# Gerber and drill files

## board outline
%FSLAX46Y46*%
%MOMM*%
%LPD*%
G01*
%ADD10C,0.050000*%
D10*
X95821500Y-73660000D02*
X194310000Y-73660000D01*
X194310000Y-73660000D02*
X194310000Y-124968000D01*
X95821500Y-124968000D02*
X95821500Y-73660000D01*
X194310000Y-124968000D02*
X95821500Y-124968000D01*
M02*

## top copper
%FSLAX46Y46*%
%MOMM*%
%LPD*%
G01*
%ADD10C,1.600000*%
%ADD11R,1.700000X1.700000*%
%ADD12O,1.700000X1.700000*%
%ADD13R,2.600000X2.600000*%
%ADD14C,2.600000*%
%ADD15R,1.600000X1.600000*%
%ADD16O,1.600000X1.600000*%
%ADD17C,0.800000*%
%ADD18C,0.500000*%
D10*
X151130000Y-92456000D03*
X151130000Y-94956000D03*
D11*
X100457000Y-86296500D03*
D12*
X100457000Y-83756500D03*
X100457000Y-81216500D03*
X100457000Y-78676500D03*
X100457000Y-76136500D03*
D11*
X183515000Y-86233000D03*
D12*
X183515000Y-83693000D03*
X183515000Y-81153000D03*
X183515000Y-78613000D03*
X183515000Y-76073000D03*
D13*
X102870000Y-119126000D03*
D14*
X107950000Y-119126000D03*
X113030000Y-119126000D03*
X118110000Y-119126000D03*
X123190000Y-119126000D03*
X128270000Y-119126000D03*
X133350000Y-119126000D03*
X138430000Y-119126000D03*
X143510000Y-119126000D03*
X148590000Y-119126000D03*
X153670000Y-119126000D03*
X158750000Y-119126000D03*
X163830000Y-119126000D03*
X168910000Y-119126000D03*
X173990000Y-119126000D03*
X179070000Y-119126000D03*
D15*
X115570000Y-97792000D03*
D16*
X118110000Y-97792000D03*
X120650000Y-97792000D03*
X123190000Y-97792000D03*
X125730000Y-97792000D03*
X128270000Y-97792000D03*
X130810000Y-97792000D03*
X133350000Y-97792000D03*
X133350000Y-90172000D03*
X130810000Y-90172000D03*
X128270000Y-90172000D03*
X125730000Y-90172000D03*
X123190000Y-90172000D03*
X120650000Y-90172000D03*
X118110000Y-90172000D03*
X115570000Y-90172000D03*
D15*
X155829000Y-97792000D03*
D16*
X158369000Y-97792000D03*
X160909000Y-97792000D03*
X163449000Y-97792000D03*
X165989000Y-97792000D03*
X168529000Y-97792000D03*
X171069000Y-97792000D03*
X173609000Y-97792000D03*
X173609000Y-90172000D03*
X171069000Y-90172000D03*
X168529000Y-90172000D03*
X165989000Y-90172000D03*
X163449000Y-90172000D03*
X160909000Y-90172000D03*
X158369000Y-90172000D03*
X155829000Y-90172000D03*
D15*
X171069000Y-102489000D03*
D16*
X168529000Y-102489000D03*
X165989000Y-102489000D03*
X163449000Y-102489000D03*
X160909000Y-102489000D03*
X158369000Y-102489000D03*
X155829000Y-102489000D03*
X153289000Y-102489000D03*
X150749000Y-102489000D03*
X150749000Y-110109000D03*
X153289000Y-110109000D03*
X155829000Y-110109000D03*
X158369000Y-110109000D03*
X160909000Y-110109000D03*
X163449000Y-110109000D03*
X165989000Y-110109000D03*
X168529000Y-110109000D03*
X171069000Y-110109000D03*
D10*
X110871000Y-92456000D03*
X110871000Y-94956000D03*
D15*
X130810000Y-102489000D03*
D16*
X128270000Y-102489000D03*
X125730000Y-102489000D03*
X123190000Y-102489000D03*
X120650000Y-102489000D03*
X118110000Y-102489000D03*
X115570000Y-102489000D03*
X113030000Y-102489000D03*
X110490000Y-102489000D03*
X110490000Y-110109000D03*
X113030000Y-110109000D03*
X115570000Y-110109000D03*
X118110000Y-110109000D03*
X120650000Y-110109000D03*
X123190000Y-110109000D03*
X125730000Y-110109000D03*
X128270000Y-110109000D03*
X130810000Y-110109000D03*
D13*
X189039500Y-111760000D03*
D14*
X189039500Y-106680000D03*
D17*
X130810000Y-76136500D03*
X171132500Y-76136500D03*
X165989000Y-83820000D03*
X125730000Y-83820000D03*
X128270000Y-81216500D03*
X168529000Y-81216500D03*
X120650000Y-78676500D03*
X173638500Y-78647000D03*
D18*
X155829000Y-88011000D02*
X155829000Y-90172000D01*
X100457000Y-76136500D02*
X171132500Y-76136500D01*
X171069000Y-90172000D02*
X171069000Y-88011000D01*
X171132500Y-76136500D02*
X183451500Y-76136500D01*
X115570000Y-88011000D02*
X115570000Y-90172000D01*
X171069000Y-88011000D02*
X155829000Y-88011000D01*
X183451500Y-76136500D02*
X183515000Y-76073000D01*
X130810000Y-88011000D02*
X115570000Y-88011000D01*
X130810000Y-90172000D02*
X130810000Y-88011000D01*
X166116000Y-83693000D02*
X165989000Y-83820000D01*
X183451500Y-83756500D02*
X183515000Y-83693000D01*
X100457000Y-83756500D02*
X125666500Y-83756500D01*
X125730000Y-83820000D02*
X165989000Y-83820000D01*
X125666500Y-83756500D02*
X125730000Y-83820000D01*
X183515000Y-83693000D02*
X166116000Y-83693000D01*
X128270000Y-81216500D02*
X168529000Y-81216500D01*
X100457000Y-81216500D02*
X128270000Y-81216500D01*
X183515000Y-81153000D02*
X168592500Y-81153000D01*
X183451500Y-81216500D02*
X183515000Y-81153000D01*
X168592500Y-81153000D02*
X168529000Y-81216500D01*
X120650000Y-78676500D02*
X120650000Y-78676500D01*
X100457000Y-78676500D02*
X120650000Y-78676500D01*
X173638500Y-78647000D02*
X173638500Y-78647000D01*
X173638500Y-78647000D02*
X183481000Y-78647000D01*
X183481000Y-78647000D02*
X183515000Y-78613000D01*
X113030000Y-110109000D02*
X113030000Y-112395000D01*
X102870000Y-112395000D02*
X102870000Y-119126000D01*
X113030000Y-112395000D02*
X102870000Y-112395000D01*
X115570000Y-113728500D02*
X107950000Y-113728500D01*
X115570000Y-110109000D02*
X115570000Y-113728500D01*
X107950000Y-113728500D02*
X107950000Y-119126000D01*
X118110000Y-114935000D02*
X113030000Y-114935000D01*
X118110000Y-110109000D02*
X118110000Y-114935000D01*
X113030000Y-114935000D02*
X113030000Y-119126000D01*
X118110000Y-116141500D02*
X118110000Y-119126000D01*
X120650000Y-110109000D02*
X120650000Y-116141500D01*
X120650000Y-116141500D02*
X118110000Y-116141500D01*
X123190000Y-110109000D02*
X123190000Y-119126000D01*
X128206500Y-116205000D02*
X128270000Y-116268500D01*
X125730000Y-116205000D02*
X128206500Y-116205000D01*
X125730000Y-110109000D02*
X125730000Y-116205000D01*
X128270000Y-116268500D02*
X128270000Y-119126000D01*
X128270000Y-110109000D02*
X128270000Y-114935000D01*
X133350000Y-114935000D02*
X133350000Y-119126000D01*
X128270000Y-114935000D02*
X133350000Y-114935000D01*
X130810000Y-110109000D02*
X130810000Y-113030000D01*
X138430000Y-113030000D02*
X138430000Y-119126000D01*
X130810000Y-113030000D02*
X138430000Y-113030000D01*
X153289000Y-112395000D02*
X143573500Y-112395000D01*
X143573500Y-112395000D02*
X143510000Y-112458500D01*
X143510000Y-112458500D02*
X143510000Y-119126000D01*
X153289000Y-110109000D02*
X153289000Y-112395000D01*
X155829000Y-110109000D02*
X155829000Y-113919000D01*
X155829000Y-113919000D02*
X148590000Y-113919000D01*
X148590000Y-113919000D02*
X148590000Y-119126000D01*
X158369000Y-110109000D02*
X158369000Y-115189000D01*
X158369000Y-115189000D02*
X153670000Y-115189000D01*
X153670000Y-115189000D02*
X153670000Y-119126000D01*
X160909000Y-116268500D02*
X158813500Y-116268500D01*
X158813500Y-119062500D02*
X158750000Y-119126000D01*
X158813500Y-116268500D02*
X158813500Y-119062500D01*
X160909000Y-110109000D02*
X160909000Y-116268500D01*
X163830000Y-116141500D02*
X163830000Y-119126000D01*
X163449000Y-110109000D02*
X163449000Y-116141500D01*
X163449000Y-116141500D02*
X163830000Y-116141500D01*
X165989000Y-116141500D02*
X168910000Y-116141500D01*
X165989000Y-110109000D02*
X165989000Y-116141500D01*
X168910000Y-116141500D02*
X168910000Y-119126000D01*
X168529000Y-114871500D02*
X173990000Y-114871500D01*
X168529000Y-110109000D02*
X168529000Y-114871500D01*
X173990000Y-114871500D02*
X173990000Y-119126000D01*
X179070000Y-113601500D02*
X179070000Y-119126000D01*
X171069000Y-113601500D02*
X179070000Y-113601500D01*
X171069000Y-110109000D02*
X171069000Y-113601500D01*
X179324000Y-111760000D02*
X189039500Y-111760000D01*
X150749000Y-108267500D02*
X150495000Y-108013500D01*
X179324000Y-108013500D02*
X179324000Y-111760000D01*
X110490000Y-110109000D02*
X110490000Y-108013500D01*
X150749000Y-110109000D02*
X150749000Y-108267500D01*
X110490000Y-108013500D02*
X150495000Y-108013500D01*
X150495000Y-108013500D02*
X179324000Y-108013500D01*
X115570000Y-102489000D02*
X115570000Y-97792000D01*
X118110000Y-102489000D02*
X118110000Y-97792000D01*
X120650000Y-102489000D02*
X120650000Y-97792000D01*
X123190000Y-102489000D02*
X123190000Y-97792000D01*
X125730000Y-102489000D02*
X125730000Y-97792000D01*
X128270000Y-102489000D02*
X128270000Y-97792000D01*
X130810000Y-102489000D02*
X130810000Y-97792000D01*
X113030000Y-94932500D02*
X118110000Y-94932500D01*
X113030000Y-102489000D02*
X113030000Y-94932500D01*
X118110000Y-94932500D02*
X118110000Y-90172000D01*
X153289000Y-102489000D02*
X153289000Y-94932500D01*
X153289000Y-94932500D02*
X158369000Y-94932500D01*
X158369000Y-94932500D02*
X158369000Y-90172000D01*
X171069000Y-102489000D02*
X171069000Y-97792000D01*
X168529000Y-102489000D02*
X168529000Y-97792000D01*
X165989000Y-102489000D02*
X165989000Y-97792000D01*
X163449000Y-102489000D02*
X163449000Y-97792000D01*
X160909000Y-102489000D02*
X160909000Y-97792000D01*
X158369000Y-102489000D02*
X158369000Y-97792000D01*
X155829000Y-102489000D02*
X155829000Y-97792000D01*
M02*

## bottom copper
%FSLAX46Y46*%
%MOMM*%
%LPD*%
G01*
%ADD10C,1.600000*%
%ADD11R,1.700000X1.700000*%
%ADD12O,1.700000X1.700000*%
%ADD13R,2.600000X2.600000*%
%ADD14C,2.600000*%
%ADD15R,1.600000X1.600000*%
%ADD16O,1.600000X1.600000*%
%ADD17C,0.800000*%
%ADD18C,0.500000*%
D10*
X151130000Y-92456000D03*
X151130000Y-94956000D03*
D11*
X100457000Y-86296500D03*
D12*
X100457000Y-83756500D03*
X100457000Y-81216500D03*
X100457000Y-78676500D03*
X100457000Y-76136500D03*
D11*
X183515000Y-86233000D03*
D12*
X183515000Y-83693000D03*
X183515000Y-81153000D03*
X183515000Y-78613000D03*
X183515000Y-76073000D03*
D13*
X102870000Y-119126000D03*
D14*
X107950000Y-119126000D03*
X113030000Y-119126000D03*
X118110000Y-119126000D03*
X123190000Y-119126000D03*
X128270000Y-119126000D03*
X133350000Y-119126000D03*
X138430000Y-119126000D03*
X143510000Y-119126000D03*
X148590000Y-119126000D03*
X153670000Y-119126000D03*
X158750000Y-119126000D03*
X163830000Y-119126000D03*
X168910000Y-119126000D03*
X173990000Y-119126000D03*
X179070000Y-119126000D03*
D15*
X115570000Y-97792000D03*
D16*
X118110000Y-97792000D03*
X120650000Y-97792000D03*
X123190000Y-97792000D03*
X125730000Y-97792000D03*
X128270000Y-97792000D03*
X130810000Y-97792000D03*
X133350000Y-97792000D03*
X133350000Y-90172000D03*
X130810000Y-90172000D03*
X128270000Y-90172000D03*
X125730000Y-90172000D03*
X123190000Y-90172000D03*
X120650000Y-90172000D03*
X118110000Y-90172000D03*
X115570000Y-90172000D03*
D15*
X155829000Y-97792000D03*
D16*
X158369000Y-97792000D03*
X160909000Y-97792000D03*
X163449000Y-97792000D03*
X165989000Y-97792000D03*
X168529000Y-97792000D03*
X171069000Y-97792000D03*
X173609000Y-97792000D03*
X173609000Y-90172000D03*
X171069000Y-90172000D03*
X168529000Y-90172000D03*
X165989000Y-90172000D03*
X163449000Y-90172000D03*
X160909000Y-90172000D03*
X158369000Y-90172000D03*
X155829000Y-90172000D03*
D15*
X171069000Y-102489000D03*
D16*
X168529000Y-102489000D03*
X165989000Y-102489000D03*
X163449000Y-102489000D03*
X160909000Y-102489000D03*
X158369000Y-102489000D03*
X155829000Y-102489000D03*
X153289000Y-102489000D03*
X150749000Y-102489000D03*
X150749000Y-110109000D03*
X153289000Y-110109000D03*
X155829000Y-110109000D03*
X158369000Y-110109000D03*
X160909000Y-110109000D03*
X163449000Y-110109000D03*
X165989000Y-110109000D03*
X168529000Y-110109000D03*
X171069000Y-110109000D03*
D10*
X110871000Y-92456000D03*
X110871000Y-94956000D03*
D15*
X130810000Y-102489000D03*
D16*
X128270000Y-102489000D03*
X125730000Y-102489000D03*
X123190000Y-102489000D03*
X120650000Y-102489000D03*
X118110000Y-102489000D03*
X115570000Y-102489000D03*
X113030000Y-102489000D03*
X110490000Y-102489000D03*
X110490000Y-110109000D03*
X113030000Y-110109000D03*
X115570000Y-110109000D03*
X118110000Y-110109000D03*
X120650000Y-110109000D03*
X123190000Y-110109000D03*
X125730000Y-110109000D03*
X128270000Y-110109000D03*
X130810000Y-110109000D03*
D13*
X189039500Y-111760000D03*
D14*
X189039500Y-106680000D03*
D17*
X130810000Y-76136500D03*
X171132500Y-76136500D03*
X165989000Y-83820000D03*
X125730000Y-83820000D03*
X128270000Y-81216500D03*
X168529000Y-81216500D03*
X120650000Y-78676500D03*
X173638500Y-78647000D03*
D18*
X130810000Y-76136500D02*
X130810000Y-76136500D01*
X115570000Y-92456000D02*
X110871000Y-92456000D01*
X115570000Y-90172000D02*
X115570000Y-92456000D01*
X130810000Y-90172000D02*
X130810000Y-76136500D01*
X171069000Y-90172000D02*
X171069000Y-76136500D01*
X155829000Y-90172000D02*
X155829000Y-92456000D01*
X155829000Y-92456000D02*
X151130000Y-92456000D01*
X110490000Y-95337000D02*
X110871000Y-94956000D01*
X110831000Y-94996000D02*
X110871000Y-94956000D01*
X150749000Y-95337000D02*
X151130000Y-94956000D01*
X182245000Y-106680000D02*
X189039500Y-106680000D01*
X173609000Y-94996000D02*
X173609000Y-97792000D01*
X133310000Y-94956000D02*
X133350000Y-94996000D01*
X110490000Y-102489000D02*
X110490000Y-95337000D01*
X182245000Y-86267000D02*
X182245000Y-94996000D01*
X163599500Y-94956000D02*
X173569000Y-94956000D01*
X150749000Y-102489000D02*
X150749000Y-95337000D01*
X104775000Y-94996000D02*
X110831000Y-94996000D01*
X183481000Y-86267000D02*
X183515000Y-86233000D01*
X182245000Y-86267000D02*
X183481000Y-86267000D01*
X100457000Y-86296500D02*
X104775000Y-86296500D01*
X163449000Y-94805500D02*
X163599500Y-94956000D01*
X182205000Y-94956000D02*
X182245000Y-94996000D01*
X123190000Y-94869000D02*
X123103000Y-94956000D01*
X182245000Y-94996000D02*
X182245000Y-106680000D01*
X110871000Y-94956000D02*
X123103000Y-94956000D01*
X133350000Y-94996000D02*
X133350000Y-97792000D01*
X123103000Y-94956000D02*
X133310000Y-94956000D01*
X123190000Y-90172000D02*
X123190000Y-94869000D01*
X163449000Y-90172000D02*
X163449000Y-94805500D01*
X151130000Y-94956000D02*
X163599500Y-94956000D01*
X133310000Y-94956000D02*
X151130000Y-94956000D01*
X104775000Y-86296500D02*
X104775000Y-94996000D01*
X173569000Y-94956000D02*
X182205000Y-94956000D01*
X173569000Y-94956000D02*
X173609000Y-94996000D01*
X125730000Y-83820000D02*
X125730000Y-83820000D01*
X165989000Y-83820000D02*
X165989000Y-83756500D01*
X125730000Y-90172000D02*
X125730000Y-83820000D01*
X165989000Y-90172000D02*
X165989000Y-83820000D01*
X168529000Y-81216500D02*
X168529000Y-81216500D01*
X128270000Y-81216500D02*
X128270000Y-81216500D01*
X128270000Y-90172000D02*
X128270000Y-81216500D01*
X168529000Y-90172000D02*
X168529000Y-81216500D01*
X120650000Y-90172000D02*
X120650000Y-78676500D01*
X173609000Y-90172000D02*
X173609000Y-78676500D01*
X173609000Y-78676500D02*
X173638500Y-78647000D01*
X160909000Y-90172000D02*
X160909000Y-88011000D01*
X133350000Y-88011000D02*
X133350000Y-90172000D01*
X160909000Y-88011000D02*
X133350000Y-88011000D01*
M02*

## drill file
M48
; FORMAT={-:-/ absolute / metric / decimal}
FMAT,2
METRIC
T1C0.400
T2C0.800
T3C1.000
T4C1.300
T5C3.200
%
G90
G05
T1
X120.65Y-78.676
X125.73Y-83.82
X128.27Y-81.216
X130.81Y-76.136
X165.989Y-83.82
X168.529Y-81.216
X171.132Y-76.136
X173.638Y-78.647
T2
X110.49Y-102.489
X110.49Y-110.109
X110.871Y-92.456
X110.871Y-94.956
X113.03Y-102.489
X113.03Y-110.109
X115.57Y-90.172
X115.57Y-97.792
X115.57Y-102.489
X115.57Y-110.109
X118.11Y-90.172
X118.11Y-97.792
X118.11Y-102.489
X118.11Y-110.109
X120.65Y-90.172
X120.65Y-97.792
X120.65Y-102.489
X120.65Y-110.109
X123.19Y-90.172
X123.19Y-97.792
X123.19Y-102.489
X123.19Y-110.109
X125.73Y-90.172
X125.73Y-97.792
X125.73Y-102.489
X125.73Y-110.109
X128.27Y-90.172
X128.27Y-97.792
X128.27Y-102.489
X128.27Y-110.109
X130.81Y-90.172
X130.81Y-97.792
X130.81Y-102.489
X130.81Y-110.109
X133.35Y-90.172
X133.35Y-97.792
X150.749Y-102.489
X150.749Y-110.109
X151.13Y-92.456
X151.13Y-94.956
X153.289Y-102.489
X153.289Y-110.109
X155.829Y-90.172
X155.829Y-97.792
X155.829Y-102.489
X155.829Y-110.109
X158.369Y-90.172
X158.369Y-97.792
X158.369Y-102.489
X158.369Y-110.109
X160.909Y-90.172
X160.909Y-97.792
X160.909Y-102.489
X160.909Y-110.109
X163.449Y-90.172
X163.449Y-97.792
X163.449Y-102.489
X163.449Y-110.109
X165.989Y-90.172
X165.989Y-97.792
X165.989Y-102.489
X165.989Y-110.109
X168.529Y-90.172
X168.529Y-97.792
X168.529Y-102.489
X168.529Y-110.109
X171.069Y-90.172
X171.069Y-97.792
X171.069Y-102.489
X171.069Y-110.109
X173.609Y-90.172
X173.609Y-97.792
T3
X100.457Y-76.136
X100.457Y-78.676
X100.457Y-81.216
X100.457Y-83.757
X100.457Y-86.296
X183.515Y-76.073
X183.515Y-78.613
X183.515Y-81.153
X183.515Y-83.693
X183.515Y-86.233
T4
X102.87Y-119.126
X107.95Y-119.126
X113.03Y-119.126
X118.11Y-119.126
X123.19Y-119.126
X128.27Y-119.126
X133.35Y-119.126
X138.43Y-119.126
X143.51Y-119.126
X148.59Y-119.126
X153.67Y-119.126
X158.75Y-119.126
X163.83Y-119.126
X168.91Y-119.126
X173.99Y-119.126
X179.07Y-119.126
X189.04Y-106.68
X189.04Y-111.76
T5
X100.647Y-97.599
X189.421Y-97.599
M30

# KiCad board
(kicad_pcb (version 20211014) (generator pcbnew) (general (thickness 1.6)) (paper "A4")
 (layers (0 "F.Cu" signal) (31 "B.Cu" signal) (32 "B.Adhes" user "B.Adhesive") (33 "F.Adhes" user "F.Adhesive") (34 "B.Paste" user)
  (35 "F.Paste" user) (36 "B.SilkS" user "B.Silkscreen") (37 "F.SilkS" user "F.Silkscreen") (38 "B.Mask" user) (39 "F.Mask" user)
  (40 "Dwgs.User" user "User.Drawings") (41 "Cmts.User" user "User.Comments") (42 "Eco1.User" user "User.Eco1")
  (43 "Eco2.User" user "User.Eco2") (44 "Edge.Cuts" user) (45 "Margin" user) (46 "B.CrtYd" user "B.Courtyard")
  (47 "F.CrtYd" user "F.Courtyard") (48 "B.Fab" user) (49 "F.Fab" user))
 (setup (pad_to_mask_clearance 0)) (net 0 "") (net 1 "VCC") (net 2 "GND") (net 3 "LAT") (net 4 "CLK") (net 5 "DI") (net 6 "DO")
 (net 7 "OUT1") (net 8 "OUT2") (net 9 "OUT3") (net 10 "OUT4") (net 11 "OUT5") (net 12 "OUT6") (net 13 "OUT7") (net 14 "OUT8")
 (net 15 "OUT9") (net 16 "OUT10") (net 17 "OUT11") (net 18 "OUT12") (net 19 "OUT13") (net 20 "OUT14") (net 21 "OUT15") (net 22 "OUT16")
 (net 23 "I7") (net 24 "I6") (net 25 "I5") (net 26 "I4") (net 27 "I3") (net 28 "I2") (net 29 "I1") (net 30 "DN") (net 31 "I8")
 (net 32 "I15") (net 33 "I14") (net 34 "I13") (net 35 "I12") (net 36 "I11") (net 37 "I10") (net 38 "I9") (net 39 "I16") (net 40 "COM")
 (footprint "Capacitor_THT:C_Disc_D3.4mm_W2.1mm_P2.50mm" (layer "F.Cu") (at 151.13 92.456 -90)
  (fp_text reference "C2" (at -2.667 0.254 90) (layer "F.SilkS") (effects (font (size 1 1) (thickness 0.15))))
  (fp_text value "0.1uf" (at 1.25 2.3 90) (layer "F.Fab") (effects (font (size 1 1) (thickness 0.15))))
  (pad "1" thru_hole circle locked (at 0 0 270) (size 1.6 1.6) (drill 0.8) (layers *.Cu *.Mask) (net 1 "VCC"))
  (pad "2" thru_hole circle locked (at 2.5 0 270) (size 1.6 1.6) (drill 0.8) (layers *.Cu *.Mask) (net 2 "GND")))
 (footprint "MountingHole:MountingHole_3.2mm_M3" (layer "F.Cu") (at 100.6475 97.5995)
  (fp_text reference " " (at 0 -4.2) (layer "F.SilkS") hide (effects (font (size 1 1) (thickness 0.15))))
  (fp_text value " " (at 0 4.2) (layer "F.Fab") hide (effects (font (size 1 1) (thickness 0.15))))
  (pad "" np_thru_hole circle locked (at 0 0) (size 3.2 3.2) (drill 3.2) (layers *.Cu *.Mask)))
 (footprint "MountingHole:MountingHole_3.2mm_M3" (layer "F.Cu") (at 189.4205 97.5995)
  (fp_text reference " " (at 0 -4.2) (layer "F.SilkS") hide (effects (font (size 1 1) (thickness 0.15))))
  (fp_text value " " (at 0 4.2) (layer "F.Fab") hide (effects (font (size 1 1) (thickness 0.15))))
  (pad "" np_thru_hole circle locked (at 0 0) (size 3.2 3.2) (drill 3.2) (layers *.Cu *.Mask)))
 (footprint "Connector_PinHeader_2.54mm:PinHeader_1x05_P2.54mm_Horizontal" (layer "F.Cu") (at 100.457 86.2965 180)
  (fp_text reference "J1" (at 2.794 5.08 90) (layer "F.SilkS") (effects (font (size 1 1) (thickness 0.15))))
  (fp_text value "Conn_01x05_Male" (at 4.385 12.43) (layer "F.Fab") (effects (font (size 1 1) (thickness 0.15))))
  (pad "1" thru_hole rect locked (at 0 0 180) (size 1.7 1.7) (drill 1) (layers *.Cu *.Mask) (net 2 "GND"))
  (pad "2" thru_hole oval locked (at 0 2.54 180) (size 1.7 1.7) (drill 1) (layers *.Cu *.Mask) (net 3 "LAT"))
  (pad "3" thru_hole oval locked (at 0 5.08 180) (size 1.7 1.7) (drill 1) (layers *.Cu *.Mask) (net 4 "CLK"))
  (pad "4" thru_hole oval locked (at 0 7.62 180) (size 1.7 1.7) (drill 1) (layers *.Cu *.Mask) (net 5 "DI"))
  (pad "5" thru_hole oval locked (at 0 10.16 180) (size 1.7 1.7) (drill 1) (layers *.Cu *.Mask) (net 1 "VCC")))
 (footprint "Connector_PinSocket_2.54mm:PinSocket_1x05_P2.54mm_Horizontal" (layer "F.Cu") (at 183.515 86.233 180)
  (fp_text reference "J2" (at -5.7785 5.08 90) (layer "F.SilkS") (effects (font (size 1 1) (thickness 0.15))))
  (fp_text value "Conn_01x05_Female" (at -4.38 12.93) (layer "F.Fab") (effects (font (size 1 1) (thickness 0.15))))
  (pad "1" thru_hole rect locked (at 0 0 180) (size 1.7 1.7) (drill 1) (layers *.Cu *.Mask) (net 2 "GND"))
  (pad "2" thru_hole oval locked (at 0 2.54 180) (size 1.7 1.7) (drill 1) (layers *.Cu *.Mask) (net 3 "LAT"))
  (pad "3" thru_hole oval locked (at 0 5.08 180) (size 1.7 1.7) (drill 1) (layers *.Cu *.Mask) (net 4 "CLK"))
  (pad "4" thru_hole oval locked (at 0 7.62 180) (size 1.7 1.7) (drill 1) (layers *.Cu *.Mask) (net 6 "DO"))
  (pad "5" thru_hole oval locked (at 0 10.16 180) (size 1.7 1.7) (drill 1) (layers *.Cu *.Mask) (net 1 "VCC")))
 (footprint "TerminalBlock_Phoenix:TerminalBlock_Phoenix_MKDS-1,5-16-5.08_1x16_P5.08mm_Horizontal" (layer "F.Cu") (at 102.87 119.126)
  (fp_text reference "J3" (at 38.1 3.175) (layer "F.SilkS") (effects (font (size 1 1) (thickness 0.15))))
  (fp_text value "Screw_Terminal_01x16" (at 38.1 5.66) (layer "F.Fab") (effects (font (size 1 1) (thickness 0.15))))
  (pad "1" thru_hole rect locked (at 0 0) (size 2.6 2.6) (drill 1.3) (layers *.Cu *.Mask) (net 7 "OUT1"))
  (pad "2" thru_hole circle locked (at 5.08 0) (size 2.6 2.6) (drill 1.3) (layers *.Cu *.Mask) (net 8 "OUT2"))
  (pad "3" thru_hole circle locked (at 10.16 0) (size 2.6 2.6) (drill 1.3) (layers *.Cu *.Mask) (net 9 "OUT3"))
  (pad "4" thru_hole circle locked (at 15.24 0) (size 2.6 2.6) (drill 1.3) (layers *.Cu *.Mask) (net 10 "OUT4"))
  (pad "5" thru_hole circle locked (at 20.32 0) (size 2.6 2.6) (drill 1.3) (layers *.Cu *.Mask) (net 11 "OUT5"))
  (pad "6" thru_hole circle locked (at 25.4 0) (size 2.6 2.6) (drill 1.3) (layers *.Cu *.Mask) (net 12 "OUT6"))
  (pad "7" thru_hole circle locked (at 30.48 0) (size 2.6 2.6) (drill 1.3) (layers *.Cu *.Mask) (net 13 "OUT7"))
  (pad "8" thru_hole circle locked (at 35.56 0) (size 2.6 2.6) (drill 1.3) (layers *.Cu *.Mask) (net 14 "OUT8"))
  (pad "9" thru_hole circle locked (at 40.64 0) (size 2.6 2.6) (drill 1.3) (layers *.Cu *.Mask) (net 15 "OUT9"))
  (pad "10" thru_hole circle locked (at 45.72 0) (size 2.6 2.6) (drill 1.3) (layers *.Cu *.Mask) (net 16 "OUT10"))
  (pad "11" thru_hole circle locked (at 50.8 0) (size 2.6 2.6) (drill 1.3) (layers *.Cu *.Mask) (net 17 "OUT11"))
  (pad "12" thru_hole circle locked (at 55.88 0) (size 2.6 2.6) (drill 1.3) (layers *.Cu *.Mask) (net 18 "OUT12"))
  (pad "13" thru_hole circle locked (at 60.96 0) (size 2.6 2.6) (drill 1.3) (layers *.Cu *.Mask) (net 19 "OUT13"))
  (pad "14" thru_hole circle locked (at 66.04 0) (size 2.6 2.6) (drill 1.3) (layers *.Cu *.Mask) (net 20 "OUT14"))
  (pad "15" thru_hole circle locked (at 71.12 0) (size 2.6 2.6) (drill 1.3) (layers *.Cu *.Mask) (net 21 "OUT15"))
  (pad "16" thru_hole circle locked (at 76.2 0) (size 2.6 2.6) (drill 1.3) (layers *.Cu *.Mask) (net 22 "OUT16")))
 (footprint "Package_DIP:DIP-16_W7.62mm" (layer "F.Cu") (at 115.57 97.792 90)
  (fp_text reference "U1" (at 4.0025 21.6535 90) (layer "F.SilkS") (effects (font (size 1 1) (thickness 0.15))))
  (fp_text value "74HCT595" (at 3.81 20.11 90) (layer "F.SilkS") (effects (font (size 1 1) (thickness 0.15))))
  (pad "1" thru_hole rect locked (at 0 0 90) (size 1.6 1.6) (drill 0.8) (layers *.Cu *.Mask) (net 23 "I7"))
  (pad "2" thru_hole oval locked (at 0 2.54 90) (size 1.6 1.6) (drill 0.8) (layers *.Cu *.Mask) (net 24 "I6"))
  (pad "3" thru_hole oval locked (at 0 5.08 90) (size 1.6 1.6) (drill 0.8) (layers *.Cu *.Mask) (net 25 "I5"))
  (pad "4" thru_hole oval locked (at 0 7.62 90) (size 1.6 1.6) (drill 0.8) (layers *.Cu *.Mask) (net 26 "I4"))
  (pad "5" thru_hole oval locked (at 0 10.16 90) (size 1.6 1.6) (drill 0.8) (layers *.Cu *.Mask) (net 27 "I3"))
  (pad "6" thru_hole oval locked (at 0 12.7 90) (size 1.6 1.6) (drill 0.8) (layers *.Cu *.Mask) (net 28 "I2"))
  (pad "7" thru_hole oval locked (at 0 15.24 90) (size 1.6 1.6) (drill 0.8) (layers *.Cu *.Mask) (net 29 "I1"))
  (pad "8" thru_hole oval locked (at 0 17.78 90) (size 1.6 1.6) (drill 0.8) (layers *.Cu *.Mask) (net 2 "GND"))
  (pad "9" thru_hole oval locked (at 7.62 17.78 90) (size 1.6 1.6) (drill 0.8) (layers *.Cu *.Mask) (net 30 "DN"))
  (pad "10" thru_hole oval locked (at 7.62 15.24 90) (size 1.6 1.6) (drill 0.8) (layers *.Cu *.Mask) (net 1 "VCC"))
  (pad "11" thru_hole oval locked (at 7.62 12.7 90) (size 1.6 1.6) (drill 0.8) (layers *.Cu *.Mask) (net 4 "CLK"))
  (pad "12" thru_hole oval locked (at 7.62 10.16 90) (size 1.6 1.6) (drill 0.8) (layers *.Cu *.Mask) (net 3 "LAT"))
  (pad "13" thru_hole oval locked (at 7.62 7.62 90) (size 1.6 1.6) (drill 0.8) (layers *.Cu *.Mask) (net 2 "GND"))
  (pad "14" thru_hole oval locked (at 7.62 5.08 90) (size 1.6 1.6) (drill 0.8) (layers *.Cu *.Mask) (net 5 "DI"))
  (pad "15" thru_hole oval locked (at 7.62 2.54 90) (size 1.6 1.6) (drill 0.8) (layers *.Cu *.Mask) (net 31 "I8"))
  (pad "16" thru_hole oval locked (at 7.62 0 90) (size 1.6 1.6) (drill 0.8) (layers *.Cu *.Mask) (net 1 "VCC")))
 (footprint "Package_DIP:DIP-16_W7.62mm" (layer "F.Cu") (at 155.829 97.792 90)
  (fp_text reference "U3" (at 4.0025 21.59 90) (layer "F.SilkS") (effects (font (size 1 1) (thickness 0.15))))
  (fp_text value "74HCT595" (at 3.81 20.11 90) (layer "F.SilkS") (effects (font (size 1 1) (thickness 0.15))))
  (pad "1" thru_hole rect locked (at 0 0 90) (size 1.6 1.6) (drill 0.8) (layers *.Cu *.Mask) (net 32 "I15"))
  (pad "2" thru_hole oval locked (at 0 2.54 90) (size 1.6 1.6) (drill 0.8) (layers *.Cu *.Mask) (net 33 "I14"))
  (pad "3" thru_hole oval locked (at 0 5.08 90) (size 1.6 1.6) (drill 0.8) (layers *.Cu *.Mask) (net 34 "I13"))
  (pad "4" thru_hole oval locked (at 0 7.62 90) (size 1.6 1.6) (drill 0.8) (layers *.Cu *.Mask) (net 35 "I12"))
  (pad "5" thru_hole oval locked (at 0 10.16 90) (size 1.6 1.6) (drill 0.8) (layers *.Cu *.Mask) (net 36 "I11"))
  (pad "6" thru_hole oval locked (at 0 12.7 90) (size 1.6 1.6) (drill 0.8) (layers *.Cu *.Mask) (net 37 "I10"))
  (pad "7" thru_hole oval locked (at 0 15.24 90) (size 1.6 1.6) (drill 0.8) (layers *.Cu *.Mask) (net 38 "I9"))
  (pad "8" thru_hole oval locked (at 0 17.78 90) (size 1.6 1.6) (drill 0.8) (layers *.Cu *.Mask) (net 2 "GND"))
  (pad "9" thru_hole oval locked (at 7.62 17.78 90) (size 1.6 1.6) (drill 0.8) (layers *.Cu *.Mask) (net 6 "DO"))
  (pad "10" thru_hole oval locked (at 7.62 15.24 90) (size 1.6 1.6) (drill 0.8) (layers *.Cu *.Mask) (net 1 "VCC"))
  (pad "11" thru_hole oval locked (at 7.62 12.7 90) (size 1.6 1.6) (drill 0.8) (layers *.Cu *.Mask) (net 4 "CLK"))
  (pad "12" thru_hole oval locked (at 7.62 10.16 90) (size 1.6 1.6) (drill 0.8) (layers *.Cu *.Mask) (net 3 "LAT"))
  (pad "13" thru_hole oval locked (at 7.62 7.62 90) (size 1.6 1.6) (drill 0.8) (layers *.Cu *.Mask) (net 2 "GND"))
  (pad "14" thru_hole oval locked (at 7.62 5.08 90) (size 1.6 1.6) (drill 0.8) (layers *.Cu *.Mask) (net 30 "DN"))
  (pad "15" thru_hole oval locked (at 7.62 2.54 90) (size 1.6 1.6) (drill 0.8) (layers *.Cu *.Mask) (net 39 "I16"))
  (pad "16" thru_hole oval locked (at 7.62 0 90) (size 1.6 1.6) (drill 0.8) (layers *.Cu *.Mask) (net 1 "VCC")))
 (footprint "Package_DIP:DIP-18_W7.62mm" (layer "F.Cu") (at 171.069 102.489 -90)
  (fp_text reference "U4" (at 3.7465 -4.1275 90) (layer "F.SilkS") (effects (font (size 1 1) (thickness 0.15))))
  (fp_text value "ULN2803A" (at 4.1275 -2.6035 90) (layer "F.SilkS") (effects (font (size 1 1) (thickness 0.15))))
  (pad "1" thru_hole rect locked (at 0 0 270) (size 1.6 1.6) (drill 0.8) (layers *.Cu *.Mask) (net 38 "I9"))
  (pad "2" thru_hole oval locked (at 0 2.54 270) (size 1.6 1.6) (drill 0.8) (layers *.Cu *.Mask) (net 37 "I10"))
  (pad "3" thru_hole oval locked (at 0 5.08 270) (size 1.6 1.6) (drill 0.8) (layers *.Cu *.Mask) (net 36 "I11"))
  (pad "4" thru_hole oval locked (at 0 7.62 270) (size 1.6 1.6) (drill 0.8) (layers *.Cu *.Mask) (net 35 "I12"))
  (pad "5" thru_hole oval locked (at 0 10.16 270) (size 1.6 1.6) (drill 0.8) (layers *.Cu *.Mask) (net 34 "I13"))
  (pad "6" thru_hole oval locked (at 0 12.7 270) (size 1.6 1.6) (drill 0.8) (layers *.Cu *.Mask) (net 33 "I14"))
  (pad "7" thru_hole oval locked (at 0 15.24 270) (size 1.6 1.6) (drill 0.8) (layers *.Cu *.Mask) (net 32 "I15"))
  (pad "8" thru_hole oval locked (at 0 17.78 270) (size 1.6 1.6) (drill 0.8) (layers *.Cu *.Mask) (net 39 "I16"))
  (pad "9" thru_hole oval locked (at 0 20.32 270) (size 1.6 1.6) (drill 0.8) (layers *.Cu *.Mask) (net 2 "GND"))
  (pad "10" thru_hole oval locked (at 7.62 20.32 270) (size 1.6 1.6) (drill 0.8) (layers *.Cu *.Mask) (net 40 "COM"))
  (pad "11" thru_hole oval locked (at 7.62 17.78 270) (size 1.6 1.6) (drill 0.8) (layers *.Cu *.Mask) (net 15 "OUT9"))
  (pad "12" thru_hole oval locked (at 7.62 15.24 270) (size 1.6 1.6) (drill 0.8) (layers *.Cu *.Mask) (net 16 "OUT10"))
  (pad "13" thru_hole oval locked (at 7.62 12.7 270) (size 1.6 1.6) (drill 0.8) (layers *.Cu *.Mask) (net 17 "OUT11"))
  (pad "14" thru_hole oval locked (at 7.62 10.16 270) (size 1.6 1.6) (drill 0.8) (layers *.Cu *.Mask) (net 18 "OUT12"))
  (pad "15" thru_hole oval locked (at 7.62 7.62 270) (size 1.6 1.6) (drill 0.8) (layers *.Cu *.Mask) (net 19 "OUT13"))
  (pad "16" thru_hole oval locked (at 7.62 5.08 270) (size 1.6 1.6) (drill 0.8) (layers *.Cu *.Mask) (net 20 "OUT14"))
  (pad "17" thru_hole oval locked (at 7.62 2.54 270) (size 1.6 1.6) (drill 0.8) (layers *.Cu *.Mask) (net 21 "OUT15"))
  (pad "18" thru_hole oval locked (at 7.62 0 270) (size 1.6 1.6) (drill 0.8) (layers *.Cu *.Mask) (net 22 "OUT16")))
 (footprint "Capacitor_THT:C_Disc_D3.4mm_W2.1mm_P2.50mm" (layer "F.Cu") (at 110.871 92.456 -90)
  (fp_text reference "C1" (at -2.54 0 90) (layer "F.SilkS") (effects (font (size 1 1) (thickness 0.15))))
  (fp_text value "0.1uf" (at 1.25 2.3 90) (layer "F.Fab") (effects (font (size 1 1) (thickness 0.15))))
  (pad "1" thru_hole circle locked (at 0 0 270) (size 1.6 1.6) (drill 0.8) (layers *.Cu *.Mask) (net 1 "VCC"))
  (pad "2" thru_hole circle locked (at 2.5 0 270) (size 1.6 1.6) (drill 0.8) (layers *.Cu *.Mask) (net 2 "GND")))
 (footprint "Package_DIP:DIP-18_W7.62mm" (layer "F.Cu") (at 130.81 102.489 -90)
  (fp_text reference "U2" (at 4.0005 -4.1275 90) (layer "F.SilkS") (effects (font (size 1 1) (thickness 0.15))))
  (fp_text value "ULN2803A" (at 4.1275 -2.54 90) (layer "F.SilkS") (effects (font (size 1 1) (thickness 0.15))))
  (pad "1" thru_hole rect locked (at 0 0 270) (size 1.6 1.6) (drill 0.8) (layers *.Cu *.Mask) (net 29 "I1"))
  (pad "2" thru_hole oval locked (at 0 2.54 270) (size 1.6 1.6) (drill 0.8) (layers *.Cu *.Mask) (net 28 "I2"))
  (pad "3" thru_hole oval locked (at 0 5.08 270) (size 1.6 1.6) (drill 0.8) (layers *.Cu *.Mask) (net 27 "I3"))
  (pad "4" thru_hole oval locked (at 0 7.62 270) (size 1.6 1.6) (drill 0.8) (layers *.Cu *.Mask) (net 26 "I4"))
  (pad "5" thru_hole oval locked (at 0 10.16 270) (size 1.6 1.6) (drill 0.8) (layers *.Cu *.Mask) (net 25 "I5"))
  (pad "6" thru_hole oval locked (at 0 12.7 270) (size 1.6 1.6) (drill 0.8) (layers *.Cu *.Mask) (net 24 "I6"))
  (pad "7" thru_hole oval locked (at 0 15.24 270) (size 1.6 1.6) (drill 0.8) (layers *.Cu *.Mask) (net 23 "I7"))
  (pad "8" thru_hole oval locked (at 0 17.78 270) (size 1.6 1.6) (drill 0.8) (layers *.Cu *.Mask) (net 31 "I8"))
  (pad "9" thru_hole oval locked (at 0 20.32 270) (size 1.6 1.6) (drill 0.8) (layers *.Cu *.Mask) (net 2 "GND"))
  (pad "10" thru_hole oval locked (at 7.62 20.32 270) (size 1.6 1.6) (drill 0.8) (layers *.Cu *.Mask) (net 40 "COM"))
  (pad "11" thru_hole oval locked (at 7.62 17.78 270) (size 1.6 1.6) (drill 0.8) (layers *.Cu *.Mask) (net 7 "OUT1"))
  (pad "12" thru_hole oval locked (at 7.62 15.24 270) (size 1.6 1.6) (drill 0.8) (layers *.Cu *.Mask) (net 8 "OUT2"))
  (pad "13" thru_hole oval locked (at 7.62 12.7 270) (size 1.6 1.6) (drill 0.8) (layers *.Cu *.Mask) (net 9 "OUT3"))
  (pad "14" thru_hole oval locked (at 7.62 10.16 270) (size 1.6 1.6) (drill 0.8) (layers *.Cu *.Mask) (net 10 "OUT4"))
  (pad "15" thru_hole oval locked (at 7.62 7.62 270) (size 1.6 1.6) (drill 0.8) (layers *.Cu *.Mask) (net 11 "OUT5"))
  (pad "16" thru_hole oval locked (at 7.62 5.08 270) (size 1.6 1.6) (drill 0.8) (layers *.Cu *.Mask) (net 12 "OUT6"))
  (pad "17" thru_hole oval locked (at 7.62 2.54 270) (size 1.6 1.6) (drill 0.8) (layers *.Cu *.Mask) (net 13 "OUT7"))
  (pad "18" thru_hole oval locked (at 7.62 0 270) (size 1.6 1.6) (drill 0.8) (layers *.Cu *.Mask) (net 14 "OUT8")))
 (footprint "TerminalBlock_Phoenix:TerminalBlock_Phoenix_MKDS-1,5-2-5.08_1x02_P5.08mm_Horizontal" (layer "F.Cu") (at 189.0395 111.76 90)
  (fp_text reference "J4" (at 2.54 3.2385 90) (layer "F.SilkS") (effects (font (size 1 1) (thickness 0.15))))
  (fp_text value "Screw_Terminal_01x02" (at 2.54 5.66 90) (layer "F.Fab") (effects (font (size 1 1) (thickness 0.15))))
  (pad "1" thru_hole rect locked (at 0 0 90) (size 2.6 2.6) (drill 1.3) (layers *.Cu *.Mask) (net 40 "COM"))
  (pad "2" thru_hole circle locked (at 5.08 0 90) (size 2.6 2.6) (drill 1.3) (layers *.Cu *.Mask) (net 2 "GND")))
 (gr_line (start 95.8215 73.66) (end 194.31 73.66) (layer "Edge.Cuts") (width 0.05))
 (gr_line (start 194.31 73.66) (end 194.31 124.968) (layer "Edge.Cuts") (width 0.05))
 (gr_line (start 95.8215 124.968) (end 95.8215 73.66) (layer "Edge.Cuts") (width 0.05))
 (gr_line (start 194.31 124.968) (end 95.8215 124.968) (layer "Edge.Cuts") (width 0.05))
 (segment (start 155.829 88.011) (end 155.829 90.172) (width 0.5) (layer "F.Cu") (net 1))
 (segment (start 100.457 76.1365) (end 171.1325 76.1365) (width 0.5) (layer "F.Cu") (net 1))
 (segment (start 171.069 90.172) (end 171.069 88.011) (width 0.5) (layer "F.Cu") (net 1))
 (segment (start 171.1325 76.1365) (end 183.4515 76.1365) (width 0.5) (layer "F.Cu") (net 1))
 (segment (start 115.57 88.011) (end 115.57 90.172) (width 0.5) (layer "F.Cu") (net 1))
 (segment (start 171.069 88.011) (end 155.829 88.011) (width 0.5) (layer "F.Cu") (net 1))
 (segment (start 183.4515 76.1365) (end 183.515 76.073) (width 0.5) (layer "F.Cu") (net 1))
 (segment (start 130.81 88.011) (end 115.57 88.011) (width 0.5) (layer "F.Cu") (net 1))
 (segment (start 130.81 90.172) (end 130.81 88.011) (width 0.5) (layer "F.Cu") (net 1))
 (via (at 130.81 76.1365) (size 0.8) (drill 0.4) (layers "F.Cu" "B.Cu") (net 1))
 (via (at 171.1325 76.1365) (size 0.8) (drill 0.4) (layers "F.Cu" "B.Cu") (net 1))
 (segment (start 130.81 76.1365) (end 130.81 76.1365) (width 0.5) (layer "B.Cu") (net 1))
 (segment (start 115.57 92.456) (end 110.871 92.456) (width 0.5) (layer "B.Cu") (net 1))
 (segment (start 115.57 90.172) (end 115.57 92.456) (width 0.5) (layer "B.Cu") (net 1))
 (segment (start 130.81 90.172) (end 130.81 76.1365) (width 0.5) (layer "B.Cu") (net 1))
 (segment (start 171.069 90.172) (end 171.069 76.1365) (width 0.5) (layer "B.Cu") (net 1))
 (segment (start 155.829 90.172) (end 155.829 92.456) (width 0.5) (layer "B.Cu") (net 1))
 (segment (start 155.829 92.456) (end 151.13 92.456) (width 0.5) (layer "B.Cu") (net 1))
 (segment (start 110.49 95.337) (end 110.871 94.956) (width 0.5) (layer "B.Cu") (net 2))
 (segment (start 110.831 94.996) (end 110.871 94.956) (width 0.5) (layer "B.Cu") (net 2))
 (segment (start 150.749 95.337) (end 151.13 94.956) (width 0.5) (layer "B.Cu") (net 2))
 (segment (start 182.245 106.68) (end 189.0395 106.68) (width 0.5) (layer "B.Cu") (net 2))
 (segment (start 173.609 94.996) (end 173.609 97.792) (width 0.5) (layer "B.Cu") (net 2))
 (segment (start 133.31 94.956) (end 133.35 94.996) (width 0.5) (layer "B.Cu") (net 2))
 (segment (start 110.49 102.489) (end 110.49 95.337) (width 0.5) (layer "B.Cu") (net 2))
 (segment (start 182.245 86.267) (end 182.245 94.996) (width 0.5) (layer "B.Cu") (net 2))
 (segment (start 163.5995 94.956) (end 173.569 94.956) (width 0.5) (layer "B.Cu") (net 2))
 (segment (start 150.749 102.489) (end 150.749 95.337) (width 0.5) (layer "B.Cu") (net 2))
 (segment (start 104.775 94.996) (end 110.831 94.996) (width 0.5) (layer "B.Cu") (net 2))
 (segment (start 183.481 86.267) (end 183.515 86.233) (width 0.5) (layer "B.Cu") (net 2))
 (segment (start 182.245 86.267) (end 183.481 86.267) (width 0.5) (layer "B.Cu") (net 2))
 (segment (start 100.457 86.2965) (end 104.775 86.2965) (width 0.5) (layer "B.Cu") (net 2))
 (segment (start 163.449 94.8055) (end 163.5995 94.956) (width 0.5) (layer "B.Cu") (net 2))
 (segment (start 182.205 94.956) (end 182.245 94.996) (width 0.5) (layer "B.Cu") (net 2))
 (segment (start 123.19 94.869) (end 123.103 94.956) (width 0.5) (layer "B.Cu") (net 2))
 (segment (start 182.245 94.996) (end 182.245 106.68) (width 0.5) (layer "B.Cu") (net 2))
 (segment (start 110.871 94.956) (end 123.103 94.956) (width 0.5) (layer "B.Cu") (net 2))
 (segment (start 133.35 94.996) (end 133.35 97.792) (width 0.5) (layer "B.Cu") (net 2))
 (segment (start 123.103 94.956) (end 133.31 94.956) (width 0.5) (layer "B.Cu") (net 2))
 (segment (start 123.19 90.172) (end 123.19 94.869) (width 0.5) (layer "B.Cu") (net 2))
 (segment (start 163.449 90.172) (end 163.449 94.8055) (width 0.5) (layer "B.Cu") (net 2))
 (segment (start 151.13 94.956) (end 163.5995 94.956) (width 0.5) (layer "B.Cu") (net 2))
 (segment (start 133.31 94.956) (end 151.13 94.956) (width 0.5) (layer "B.Cu") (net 2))
 (segment (start 104.775 86.2965) (end 104.775 94.996) (width 0.5) (layer "B.Cu") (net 2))
 (segment (start 173.569 94.956) (end 182.205 94.956) (width 0.5) (layer "B.Cu") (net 2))
 (segment (start 173.569 94.956) (end 173.609 94.996) (width 0.5) (layer "B.Cu") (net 2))
 (segment (start 166.116 83.693) (end 165.989 83.82) (width 0.5) (layer "F.Cu") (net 3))
 (segment (start 183.4515 83.7565) (end 183.515 83.693) (width 0.5) (layer "F.Cu") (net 3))
 (segment (start 100.457 83.7565) (end 125.6665 83.7565) (width 0.5) (layer "F.Cu") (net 3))
 (segment (start 125.73 83.82) (end 165.989 83.82) (width 0.5) (layer "F.Cu") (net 3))
 (segment (start 125.6665 83.7565) (end 125.73 83.82) (width 0.5) (layer "F.Cu") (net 3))
 (segment (start 183.515 83.693) (end 166.116 83.693) (width 0.5) (layer "F.Cu") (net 3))
 (via (at 165.989 83.82) (size 0.8) (drill 0.4) (layers "F.Cu" "B.Cu") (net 3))
 (via (at 125.73 83.82) (size 0.8) (drill 0.4) (layers "F.Cu" "B.Cu") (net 3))
 (segment (start 125.73 83.82) (end 125.73 83.82) (width 0.5) (layer "B.Cu") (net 3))
 (segment (start 165.989 83.82) (end 165.989 83.7565) (width 0.5) (layer "B.Cu") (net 3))
 (segment (start 125.73 90.172) (end 125.73 83.82) (width 0.5) (layer "B.Cu") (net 3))
 (segment (start 165.989 90.172) (end 165.989 83.82) (width 0.5) (layer "B.Cu") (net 3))
 (segment (start 128.27 81.2165) (end 168.529 81.2165) (width 0.5) (layer "F.Cu") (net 4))
 (segment (start 100.457 81.2165) (end 128.27 81.2165) (width 0.5) (layer "F.Cu") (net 4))
 (segment (start 183.515 81.153) (end 168.5925 81.153) (width 0.5) (layer "F.Cu") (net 4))
 (segment (start 183.4515 81.2165) (end 183.515 81.153) (width 0.5) (layer "F.Cu") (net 4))
 (segment (start 168.5925 81.153) (end 168.529 81.2165) (width 0.5) (layer "F.Cu") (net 4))
 (via (at 128.27 81.2165) (size 0.8) (drill 0.4) (layers "F.Cu" "B.Cu") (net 4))
 (via (at 168.529 81.2165) (size 0.8) (drill 0.4) (layers "F.Cu" "B.Cu") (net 4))
 (segment (start 168.529 81.2165) (end 168.529 81.2165) (width 0.5) (layer "B.Cu") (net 4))
 (segment (start 128.27 81.2165) (end 128.27 81.2165) (width 0.5) (layer "B.Cu") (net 4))
 (segment (start 128.27 90.172) (end 128.27 81.2165) (width 0.5) (layer "B.Cu") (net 4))
 (segment (start 168.529 90.172) (end 168.529 81.2165) (width 0.5) (layer "B.Cu") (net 4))
 (segment (start 120.65 78.6765) (end 120.65 78.6765) (width 0.5) (layer "F.Cu") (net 5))
 (segment (start 100.457 78.6765) (end 120.65 78.6765) (width 0.5) (layer "F.Cu") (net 5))
 (via (at 120.65 78.6765) (size 0.8) (drill 0.4) (layers "F.Cu" "B.Cu") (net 5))
 (segment (start 120.65 90.172) (end 120.65 78.6765) (width 0.5) (layer "B.Cu") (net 5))
 (segment (start 173.6385 78.647) (end 173.6385 78.647) (width 0.5) (layer "F.Cu") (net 6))
 (segment (start 173.6385 78.647) (end 183.481 78.647) (width 0.5) (layer "F.Cu") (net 6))
 (segment (start 183.481 78.647) (end 183.515 78.613) (width 0.5) (layer "F.Cu") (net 6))
 (via (at 173.6385 78.647) (size 0.8) (drill 0.4) (layers "F.Cu" "B.Cu") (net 6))
 (segment (start 173.609 90.172) (end 173.609 78.6765) (width 0.5) (layer "B.Cu") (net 6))
 (segment (start 173.609 78.6765) (end 173.6385 78.647) (width 0.5) (layer "B.Cu") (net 6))
 (segment (start 113.03 110.109) (end 113.03 112.395) (width 0.5) (layer "F.Cu") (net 7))
 (segment (start 102.87 112.395) (end 102.87 119.126) (width 0.5) (layer "F.Cu") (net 7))
 (segment (start 113.03 112.395) (end 102.87 112.395) (width 0.5) (layer "F.Cu") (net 7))
 (segment (start 115.57 113.7285) (end 107.95 113.7285) (width 0.5) (layer "F.Cu") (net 8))
 (segment (start 115.57 110.109) (end 115.57 113.7285) (width 0.5) (layer "F.Cu") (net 8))
 (segment (start 107.95 113.7285) (end 107.95 119.126) (width 0.5) (layer "F.Cu") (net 8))
 (segment (start 118.11 114.935) (end 113.03 114.935) (width 0.5) (layer "F.Cu") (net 9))
 (segment (start 118.11 110.109) (end 118.11 114.935) (width 0.5) (layer "F.Cu") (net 9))
 (segment (start 113.03 114.935) (end 113.03 119.126) (width 0.5) (layer "F.Cu") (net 9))
 (segment (start 118.11 116.1415) (end 118.11 119.126) (width 0.5) (layer "F.Cu") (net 10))
 (segment (start 120.65 110.109) (end 120.65 116.1415) (width 0.5) (layer "F.Cu") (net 10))
 (segment (start 120.65 116.1415) (end 118.11 116.1415) (width 0.5) (layer "F.Cu") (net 10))
 (segment (start 123.19 110.109) (end 123.19 119.126) (width 0.5) (layer "F.Cu") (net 11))
 (segment (start 128.2065 116.205) (end 128.27 116.2685) (width 0.5) (layer "F.Cu") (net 12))
 (segment (start 125.73 116.205) (end 128.2065 116.205) (width 0.5) (layer "F.Cu") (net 12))
 (segment (start 125.73 110.109) (end 125.73 116.205) (width 0.5) (layer "F.Cu") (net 12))
 (segment (start 128.27 116.2685) (end 128.27 119.126) (width 0.5) (layer "F.Cu") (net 12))
 (segment (start 128.27 110.109) (end 128.27 114.935) (width 0.5) (layer "F.Cu") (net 13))
 (segment (start 133.35 114.935) (end 133.35 119.126) (width 0.5) (layer "F.Cu") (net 13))
 (segment (start 128.27 114.935) (end 133.35 114.935) (width 0.5) (layer "F.Cu") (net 13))
 (segment (start 130.81 110.109) (end 130.81 113.03) (width 0.5) (layer "F.Cu") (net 14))
 (segment (start 138.43 113.03) (end 138.43 119.126) (width 0.5) (layer "F.Cu") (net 14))
 (segment (start 130.81 113.03) (end 138.43 113.03) (width 0.5) (layer "F.Cu") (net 14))
 (segment (start 153.289 112.395) (end 143.5735 112.395) (width 0.5) (layer "F.Cu") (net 15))
 (segment (start 143.5735 112.395) (end 143.51 112.4585) (width 0.5) (layer "F.Cu") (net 15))
 (segment (start 143.51 112.4585) (end 143.51 119.126) (width 0.5) (layer "F.Cu") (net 15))
 (segment (start 153.289 110.109) (end 153.289 112.395) (width 0.5) (layer "F.Cu") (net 15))
 (segment (start 155.829 110.109) (end 155.829 113.919) (width 0.5) (layer "F.Cu") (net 16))
 (segment (start 155.829 113.919) (end 148.59 113.919) (width 0.5) (layer "F.Cu") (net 16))
 (segment (start 148.59 113.919) (end 148.59 119.126) (width 0.5) (layer "F.Cu") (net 16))
 (segment (start 158.369 110.109) (end 158.369 115.189) (width 0.5) (layer "F.Cu") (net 17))
 (segment (start 158.369 115.189) (end 153.67 115.189) (width 0.5) (layer "F.Cu") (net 17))
 (segment (start 153.67 115.189) (end 153.67 119.126) (width 0.5) (layer "F.Cu") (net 17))
 (segment (start 160.909 116.2685) (end 158.8135 116.2685) (width 0.5) (layer "F.Cu") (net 18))
 (segment (start 158.8135 119.0625) (end 158.75 119.126) (width 0.5) (layer "F.Cu") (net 18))
 (segment (start 158.8135 116.2685) (end 158.8135 119.0625) (width 0.5) (layer "F.Cu") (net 18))
 (segment (start 160.909 110.109) (end 160.909 116.2685) (width 0.5) (layer "F.Cu") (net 18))
 (segment (start 163.83 116.1415) (end 163.83 119.126) (width 0.5) (layer "F.Cu") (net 19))
 (segment (start 163.449 110.109) (end 163.449 116.1415) (width 0.5) (layer "F.Cu") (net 19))
 (segment (start 163.449 116.1415) (end 163.83 116.1415) (width 0.5) (layer "F.Cu") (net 19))
 (segment (start 165.989 116.1415) (end 168.91 116.1415) (width 0.5) (layer "F.Cu") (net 20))
 (segment (start 165.989 110.109) (end 165.989 116.1415) (width 0.5) (layer "F.Cu") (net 20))
 (segment (start 168.91 116.1415) (end 168.91 119.126) (width 0.5) (layer "F.Cu") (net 20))
 (segment (start 168.529 114.8715) (end 173.99 114.8715) (width 0.5) (layer "F.Cu") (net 21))
 (segment (start 168.529 110.109) (end 168.529 114.8715) (width 0.5) (layer "F.Cu") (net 21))
 (segment (start 173.99 114.8715) (end 173.99 119.126) (width 0.5) (layer "F.Cu") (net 21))
 (segment (start 179.07 113.6015) (end 179.07 119.126) (width 0.5) (layer "F.Cu") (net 22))
 (segment (start 171.069 113.6015) (end 179.07 113.6015) (width 0.5) (layer "F.Cu") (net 22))
 (segment (start 171.069 110.109) (end 171.069 113.6015) (width 0.5) (layer "F.Cu") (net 22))
 (segment (start 179.324 111.76) (end 189.0395 111.76) (width 0.5) (layer "F.Cu") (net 40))
 (segment (start 150.749 108.2675) (end 150.495 108.0135) (width 0.5) (layer "F.Cu") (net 40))
 (segment (start 179.324 108.0135) (end 179.324 111.76) (width 0.5) (layer "F.Cu") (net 40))
 (segment (start 110.49 110.109) (end 110.49 108.0135) (width 0.5) (layer "F.Cu") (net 40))
 (segment (start 150.749 110.109) (end 150.749 108.2675) (width 0.5) (layer "F.Cu") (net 40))
 (segment (start 110.49 108.0135) (end 150.495 108.0135) (width 0.5) (layer "F.Cu") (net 40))
 (segment (start 150.495 108.0135) (end 179.324 108.0135) (width 0.5) (layer "F.Cu") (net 40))
 (segment (start 160.909 90.172) (end 160.909 88.011) (width 0.5) (layer "B.Cu") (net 30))
 (segment (start 133.35 88.011) (end 133.35 90.172) (width 0.5) (layer "B.Cu") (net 30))
 (segment (start 160.909 88.011) (end 133.35 88.011) (width 0.5) (layer "B.Cu") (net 30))
 (segment (start 115.57 102.489) (end 115.57 97.792) (width 0.5) (layer "F.Cu") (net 23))
 (segment (start 118.11 102.489) (end 118.11 97.792) (width 0.5) (layer "F.Cu") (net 24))
 (segment (start 120.65 102.489) (end 120.65 97.792) (width 0.5) (layer "F.Cu") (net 25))
 (segment (start 123.19 102.489) (end 123.19 97.792) (width 0.5) (layer "F.Cu") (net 26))
 (segment (start 125.73 102.489) (end 125.73 97.792) (width 0.5) (layer "F.Cu") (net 27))
 (segment (start 128.27 102.489) (end 128.27 97.792) (width 0.5) (layer "F.Cu") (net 28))
 (segment (start 130.81 102.489) (end 130.81 97.792) (width 0.5) (layer "F.Cu") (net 29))
 (segment (start 113.03 94.9325) (end 118.11 94.9325) (width 0.5) (layer "F.Cu") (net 31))
 (segment (start 113.03 102.489) (end 113.03 94.9325) (width 0.5) (layer "F.Cu") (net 31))
 (segment (start 118.11 94.9325) (end 118.11 90.172) (width 0.5) (layer "F.Cu") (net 31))
 (segment (start 153.289 102.489) (end 153.289 94.9325) (width 0.5) (layer "F.Cu") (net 39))
 (segment (start 153.289 94.9325) (end 158.369 94.9325) (width 0.5) (layer "F.Cu") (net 39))
 (segment (start 158.369 94.9325) (end 158.369 90.172) (width 0.5) (layer "F.Cu") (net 39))
 (segment (start 171.069 102.489) (end 171.069 97.792) (width 0.5) (layer "F.Cu") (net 38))
 (segment (start 168.529 102.489) (end 168.529 97.792) (width 0.5) (layer "F.Cu") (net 37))
 (segment (start 165.989 102.489) (end 165.989 97.792) (width 0.5) (layer "F.Cu") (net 36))
 (segment (start 163.449 102.489) (end 163.449 97.792) (width 0.5) (layer "F.Cu") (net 35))
 (segment (start 160.909 102.489) (end 160.909 97.792) (width 0.5) (layer "F.Cu") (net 34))
 (segment (start 158.369 102.489) (end 158.369 97.792) (width 0.5) (layer "F.Cu") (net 33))
 (segment (start 155.829 102.489) (end 155.829 97.792) (width 0.5) (layer "F.Cu") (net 32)))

